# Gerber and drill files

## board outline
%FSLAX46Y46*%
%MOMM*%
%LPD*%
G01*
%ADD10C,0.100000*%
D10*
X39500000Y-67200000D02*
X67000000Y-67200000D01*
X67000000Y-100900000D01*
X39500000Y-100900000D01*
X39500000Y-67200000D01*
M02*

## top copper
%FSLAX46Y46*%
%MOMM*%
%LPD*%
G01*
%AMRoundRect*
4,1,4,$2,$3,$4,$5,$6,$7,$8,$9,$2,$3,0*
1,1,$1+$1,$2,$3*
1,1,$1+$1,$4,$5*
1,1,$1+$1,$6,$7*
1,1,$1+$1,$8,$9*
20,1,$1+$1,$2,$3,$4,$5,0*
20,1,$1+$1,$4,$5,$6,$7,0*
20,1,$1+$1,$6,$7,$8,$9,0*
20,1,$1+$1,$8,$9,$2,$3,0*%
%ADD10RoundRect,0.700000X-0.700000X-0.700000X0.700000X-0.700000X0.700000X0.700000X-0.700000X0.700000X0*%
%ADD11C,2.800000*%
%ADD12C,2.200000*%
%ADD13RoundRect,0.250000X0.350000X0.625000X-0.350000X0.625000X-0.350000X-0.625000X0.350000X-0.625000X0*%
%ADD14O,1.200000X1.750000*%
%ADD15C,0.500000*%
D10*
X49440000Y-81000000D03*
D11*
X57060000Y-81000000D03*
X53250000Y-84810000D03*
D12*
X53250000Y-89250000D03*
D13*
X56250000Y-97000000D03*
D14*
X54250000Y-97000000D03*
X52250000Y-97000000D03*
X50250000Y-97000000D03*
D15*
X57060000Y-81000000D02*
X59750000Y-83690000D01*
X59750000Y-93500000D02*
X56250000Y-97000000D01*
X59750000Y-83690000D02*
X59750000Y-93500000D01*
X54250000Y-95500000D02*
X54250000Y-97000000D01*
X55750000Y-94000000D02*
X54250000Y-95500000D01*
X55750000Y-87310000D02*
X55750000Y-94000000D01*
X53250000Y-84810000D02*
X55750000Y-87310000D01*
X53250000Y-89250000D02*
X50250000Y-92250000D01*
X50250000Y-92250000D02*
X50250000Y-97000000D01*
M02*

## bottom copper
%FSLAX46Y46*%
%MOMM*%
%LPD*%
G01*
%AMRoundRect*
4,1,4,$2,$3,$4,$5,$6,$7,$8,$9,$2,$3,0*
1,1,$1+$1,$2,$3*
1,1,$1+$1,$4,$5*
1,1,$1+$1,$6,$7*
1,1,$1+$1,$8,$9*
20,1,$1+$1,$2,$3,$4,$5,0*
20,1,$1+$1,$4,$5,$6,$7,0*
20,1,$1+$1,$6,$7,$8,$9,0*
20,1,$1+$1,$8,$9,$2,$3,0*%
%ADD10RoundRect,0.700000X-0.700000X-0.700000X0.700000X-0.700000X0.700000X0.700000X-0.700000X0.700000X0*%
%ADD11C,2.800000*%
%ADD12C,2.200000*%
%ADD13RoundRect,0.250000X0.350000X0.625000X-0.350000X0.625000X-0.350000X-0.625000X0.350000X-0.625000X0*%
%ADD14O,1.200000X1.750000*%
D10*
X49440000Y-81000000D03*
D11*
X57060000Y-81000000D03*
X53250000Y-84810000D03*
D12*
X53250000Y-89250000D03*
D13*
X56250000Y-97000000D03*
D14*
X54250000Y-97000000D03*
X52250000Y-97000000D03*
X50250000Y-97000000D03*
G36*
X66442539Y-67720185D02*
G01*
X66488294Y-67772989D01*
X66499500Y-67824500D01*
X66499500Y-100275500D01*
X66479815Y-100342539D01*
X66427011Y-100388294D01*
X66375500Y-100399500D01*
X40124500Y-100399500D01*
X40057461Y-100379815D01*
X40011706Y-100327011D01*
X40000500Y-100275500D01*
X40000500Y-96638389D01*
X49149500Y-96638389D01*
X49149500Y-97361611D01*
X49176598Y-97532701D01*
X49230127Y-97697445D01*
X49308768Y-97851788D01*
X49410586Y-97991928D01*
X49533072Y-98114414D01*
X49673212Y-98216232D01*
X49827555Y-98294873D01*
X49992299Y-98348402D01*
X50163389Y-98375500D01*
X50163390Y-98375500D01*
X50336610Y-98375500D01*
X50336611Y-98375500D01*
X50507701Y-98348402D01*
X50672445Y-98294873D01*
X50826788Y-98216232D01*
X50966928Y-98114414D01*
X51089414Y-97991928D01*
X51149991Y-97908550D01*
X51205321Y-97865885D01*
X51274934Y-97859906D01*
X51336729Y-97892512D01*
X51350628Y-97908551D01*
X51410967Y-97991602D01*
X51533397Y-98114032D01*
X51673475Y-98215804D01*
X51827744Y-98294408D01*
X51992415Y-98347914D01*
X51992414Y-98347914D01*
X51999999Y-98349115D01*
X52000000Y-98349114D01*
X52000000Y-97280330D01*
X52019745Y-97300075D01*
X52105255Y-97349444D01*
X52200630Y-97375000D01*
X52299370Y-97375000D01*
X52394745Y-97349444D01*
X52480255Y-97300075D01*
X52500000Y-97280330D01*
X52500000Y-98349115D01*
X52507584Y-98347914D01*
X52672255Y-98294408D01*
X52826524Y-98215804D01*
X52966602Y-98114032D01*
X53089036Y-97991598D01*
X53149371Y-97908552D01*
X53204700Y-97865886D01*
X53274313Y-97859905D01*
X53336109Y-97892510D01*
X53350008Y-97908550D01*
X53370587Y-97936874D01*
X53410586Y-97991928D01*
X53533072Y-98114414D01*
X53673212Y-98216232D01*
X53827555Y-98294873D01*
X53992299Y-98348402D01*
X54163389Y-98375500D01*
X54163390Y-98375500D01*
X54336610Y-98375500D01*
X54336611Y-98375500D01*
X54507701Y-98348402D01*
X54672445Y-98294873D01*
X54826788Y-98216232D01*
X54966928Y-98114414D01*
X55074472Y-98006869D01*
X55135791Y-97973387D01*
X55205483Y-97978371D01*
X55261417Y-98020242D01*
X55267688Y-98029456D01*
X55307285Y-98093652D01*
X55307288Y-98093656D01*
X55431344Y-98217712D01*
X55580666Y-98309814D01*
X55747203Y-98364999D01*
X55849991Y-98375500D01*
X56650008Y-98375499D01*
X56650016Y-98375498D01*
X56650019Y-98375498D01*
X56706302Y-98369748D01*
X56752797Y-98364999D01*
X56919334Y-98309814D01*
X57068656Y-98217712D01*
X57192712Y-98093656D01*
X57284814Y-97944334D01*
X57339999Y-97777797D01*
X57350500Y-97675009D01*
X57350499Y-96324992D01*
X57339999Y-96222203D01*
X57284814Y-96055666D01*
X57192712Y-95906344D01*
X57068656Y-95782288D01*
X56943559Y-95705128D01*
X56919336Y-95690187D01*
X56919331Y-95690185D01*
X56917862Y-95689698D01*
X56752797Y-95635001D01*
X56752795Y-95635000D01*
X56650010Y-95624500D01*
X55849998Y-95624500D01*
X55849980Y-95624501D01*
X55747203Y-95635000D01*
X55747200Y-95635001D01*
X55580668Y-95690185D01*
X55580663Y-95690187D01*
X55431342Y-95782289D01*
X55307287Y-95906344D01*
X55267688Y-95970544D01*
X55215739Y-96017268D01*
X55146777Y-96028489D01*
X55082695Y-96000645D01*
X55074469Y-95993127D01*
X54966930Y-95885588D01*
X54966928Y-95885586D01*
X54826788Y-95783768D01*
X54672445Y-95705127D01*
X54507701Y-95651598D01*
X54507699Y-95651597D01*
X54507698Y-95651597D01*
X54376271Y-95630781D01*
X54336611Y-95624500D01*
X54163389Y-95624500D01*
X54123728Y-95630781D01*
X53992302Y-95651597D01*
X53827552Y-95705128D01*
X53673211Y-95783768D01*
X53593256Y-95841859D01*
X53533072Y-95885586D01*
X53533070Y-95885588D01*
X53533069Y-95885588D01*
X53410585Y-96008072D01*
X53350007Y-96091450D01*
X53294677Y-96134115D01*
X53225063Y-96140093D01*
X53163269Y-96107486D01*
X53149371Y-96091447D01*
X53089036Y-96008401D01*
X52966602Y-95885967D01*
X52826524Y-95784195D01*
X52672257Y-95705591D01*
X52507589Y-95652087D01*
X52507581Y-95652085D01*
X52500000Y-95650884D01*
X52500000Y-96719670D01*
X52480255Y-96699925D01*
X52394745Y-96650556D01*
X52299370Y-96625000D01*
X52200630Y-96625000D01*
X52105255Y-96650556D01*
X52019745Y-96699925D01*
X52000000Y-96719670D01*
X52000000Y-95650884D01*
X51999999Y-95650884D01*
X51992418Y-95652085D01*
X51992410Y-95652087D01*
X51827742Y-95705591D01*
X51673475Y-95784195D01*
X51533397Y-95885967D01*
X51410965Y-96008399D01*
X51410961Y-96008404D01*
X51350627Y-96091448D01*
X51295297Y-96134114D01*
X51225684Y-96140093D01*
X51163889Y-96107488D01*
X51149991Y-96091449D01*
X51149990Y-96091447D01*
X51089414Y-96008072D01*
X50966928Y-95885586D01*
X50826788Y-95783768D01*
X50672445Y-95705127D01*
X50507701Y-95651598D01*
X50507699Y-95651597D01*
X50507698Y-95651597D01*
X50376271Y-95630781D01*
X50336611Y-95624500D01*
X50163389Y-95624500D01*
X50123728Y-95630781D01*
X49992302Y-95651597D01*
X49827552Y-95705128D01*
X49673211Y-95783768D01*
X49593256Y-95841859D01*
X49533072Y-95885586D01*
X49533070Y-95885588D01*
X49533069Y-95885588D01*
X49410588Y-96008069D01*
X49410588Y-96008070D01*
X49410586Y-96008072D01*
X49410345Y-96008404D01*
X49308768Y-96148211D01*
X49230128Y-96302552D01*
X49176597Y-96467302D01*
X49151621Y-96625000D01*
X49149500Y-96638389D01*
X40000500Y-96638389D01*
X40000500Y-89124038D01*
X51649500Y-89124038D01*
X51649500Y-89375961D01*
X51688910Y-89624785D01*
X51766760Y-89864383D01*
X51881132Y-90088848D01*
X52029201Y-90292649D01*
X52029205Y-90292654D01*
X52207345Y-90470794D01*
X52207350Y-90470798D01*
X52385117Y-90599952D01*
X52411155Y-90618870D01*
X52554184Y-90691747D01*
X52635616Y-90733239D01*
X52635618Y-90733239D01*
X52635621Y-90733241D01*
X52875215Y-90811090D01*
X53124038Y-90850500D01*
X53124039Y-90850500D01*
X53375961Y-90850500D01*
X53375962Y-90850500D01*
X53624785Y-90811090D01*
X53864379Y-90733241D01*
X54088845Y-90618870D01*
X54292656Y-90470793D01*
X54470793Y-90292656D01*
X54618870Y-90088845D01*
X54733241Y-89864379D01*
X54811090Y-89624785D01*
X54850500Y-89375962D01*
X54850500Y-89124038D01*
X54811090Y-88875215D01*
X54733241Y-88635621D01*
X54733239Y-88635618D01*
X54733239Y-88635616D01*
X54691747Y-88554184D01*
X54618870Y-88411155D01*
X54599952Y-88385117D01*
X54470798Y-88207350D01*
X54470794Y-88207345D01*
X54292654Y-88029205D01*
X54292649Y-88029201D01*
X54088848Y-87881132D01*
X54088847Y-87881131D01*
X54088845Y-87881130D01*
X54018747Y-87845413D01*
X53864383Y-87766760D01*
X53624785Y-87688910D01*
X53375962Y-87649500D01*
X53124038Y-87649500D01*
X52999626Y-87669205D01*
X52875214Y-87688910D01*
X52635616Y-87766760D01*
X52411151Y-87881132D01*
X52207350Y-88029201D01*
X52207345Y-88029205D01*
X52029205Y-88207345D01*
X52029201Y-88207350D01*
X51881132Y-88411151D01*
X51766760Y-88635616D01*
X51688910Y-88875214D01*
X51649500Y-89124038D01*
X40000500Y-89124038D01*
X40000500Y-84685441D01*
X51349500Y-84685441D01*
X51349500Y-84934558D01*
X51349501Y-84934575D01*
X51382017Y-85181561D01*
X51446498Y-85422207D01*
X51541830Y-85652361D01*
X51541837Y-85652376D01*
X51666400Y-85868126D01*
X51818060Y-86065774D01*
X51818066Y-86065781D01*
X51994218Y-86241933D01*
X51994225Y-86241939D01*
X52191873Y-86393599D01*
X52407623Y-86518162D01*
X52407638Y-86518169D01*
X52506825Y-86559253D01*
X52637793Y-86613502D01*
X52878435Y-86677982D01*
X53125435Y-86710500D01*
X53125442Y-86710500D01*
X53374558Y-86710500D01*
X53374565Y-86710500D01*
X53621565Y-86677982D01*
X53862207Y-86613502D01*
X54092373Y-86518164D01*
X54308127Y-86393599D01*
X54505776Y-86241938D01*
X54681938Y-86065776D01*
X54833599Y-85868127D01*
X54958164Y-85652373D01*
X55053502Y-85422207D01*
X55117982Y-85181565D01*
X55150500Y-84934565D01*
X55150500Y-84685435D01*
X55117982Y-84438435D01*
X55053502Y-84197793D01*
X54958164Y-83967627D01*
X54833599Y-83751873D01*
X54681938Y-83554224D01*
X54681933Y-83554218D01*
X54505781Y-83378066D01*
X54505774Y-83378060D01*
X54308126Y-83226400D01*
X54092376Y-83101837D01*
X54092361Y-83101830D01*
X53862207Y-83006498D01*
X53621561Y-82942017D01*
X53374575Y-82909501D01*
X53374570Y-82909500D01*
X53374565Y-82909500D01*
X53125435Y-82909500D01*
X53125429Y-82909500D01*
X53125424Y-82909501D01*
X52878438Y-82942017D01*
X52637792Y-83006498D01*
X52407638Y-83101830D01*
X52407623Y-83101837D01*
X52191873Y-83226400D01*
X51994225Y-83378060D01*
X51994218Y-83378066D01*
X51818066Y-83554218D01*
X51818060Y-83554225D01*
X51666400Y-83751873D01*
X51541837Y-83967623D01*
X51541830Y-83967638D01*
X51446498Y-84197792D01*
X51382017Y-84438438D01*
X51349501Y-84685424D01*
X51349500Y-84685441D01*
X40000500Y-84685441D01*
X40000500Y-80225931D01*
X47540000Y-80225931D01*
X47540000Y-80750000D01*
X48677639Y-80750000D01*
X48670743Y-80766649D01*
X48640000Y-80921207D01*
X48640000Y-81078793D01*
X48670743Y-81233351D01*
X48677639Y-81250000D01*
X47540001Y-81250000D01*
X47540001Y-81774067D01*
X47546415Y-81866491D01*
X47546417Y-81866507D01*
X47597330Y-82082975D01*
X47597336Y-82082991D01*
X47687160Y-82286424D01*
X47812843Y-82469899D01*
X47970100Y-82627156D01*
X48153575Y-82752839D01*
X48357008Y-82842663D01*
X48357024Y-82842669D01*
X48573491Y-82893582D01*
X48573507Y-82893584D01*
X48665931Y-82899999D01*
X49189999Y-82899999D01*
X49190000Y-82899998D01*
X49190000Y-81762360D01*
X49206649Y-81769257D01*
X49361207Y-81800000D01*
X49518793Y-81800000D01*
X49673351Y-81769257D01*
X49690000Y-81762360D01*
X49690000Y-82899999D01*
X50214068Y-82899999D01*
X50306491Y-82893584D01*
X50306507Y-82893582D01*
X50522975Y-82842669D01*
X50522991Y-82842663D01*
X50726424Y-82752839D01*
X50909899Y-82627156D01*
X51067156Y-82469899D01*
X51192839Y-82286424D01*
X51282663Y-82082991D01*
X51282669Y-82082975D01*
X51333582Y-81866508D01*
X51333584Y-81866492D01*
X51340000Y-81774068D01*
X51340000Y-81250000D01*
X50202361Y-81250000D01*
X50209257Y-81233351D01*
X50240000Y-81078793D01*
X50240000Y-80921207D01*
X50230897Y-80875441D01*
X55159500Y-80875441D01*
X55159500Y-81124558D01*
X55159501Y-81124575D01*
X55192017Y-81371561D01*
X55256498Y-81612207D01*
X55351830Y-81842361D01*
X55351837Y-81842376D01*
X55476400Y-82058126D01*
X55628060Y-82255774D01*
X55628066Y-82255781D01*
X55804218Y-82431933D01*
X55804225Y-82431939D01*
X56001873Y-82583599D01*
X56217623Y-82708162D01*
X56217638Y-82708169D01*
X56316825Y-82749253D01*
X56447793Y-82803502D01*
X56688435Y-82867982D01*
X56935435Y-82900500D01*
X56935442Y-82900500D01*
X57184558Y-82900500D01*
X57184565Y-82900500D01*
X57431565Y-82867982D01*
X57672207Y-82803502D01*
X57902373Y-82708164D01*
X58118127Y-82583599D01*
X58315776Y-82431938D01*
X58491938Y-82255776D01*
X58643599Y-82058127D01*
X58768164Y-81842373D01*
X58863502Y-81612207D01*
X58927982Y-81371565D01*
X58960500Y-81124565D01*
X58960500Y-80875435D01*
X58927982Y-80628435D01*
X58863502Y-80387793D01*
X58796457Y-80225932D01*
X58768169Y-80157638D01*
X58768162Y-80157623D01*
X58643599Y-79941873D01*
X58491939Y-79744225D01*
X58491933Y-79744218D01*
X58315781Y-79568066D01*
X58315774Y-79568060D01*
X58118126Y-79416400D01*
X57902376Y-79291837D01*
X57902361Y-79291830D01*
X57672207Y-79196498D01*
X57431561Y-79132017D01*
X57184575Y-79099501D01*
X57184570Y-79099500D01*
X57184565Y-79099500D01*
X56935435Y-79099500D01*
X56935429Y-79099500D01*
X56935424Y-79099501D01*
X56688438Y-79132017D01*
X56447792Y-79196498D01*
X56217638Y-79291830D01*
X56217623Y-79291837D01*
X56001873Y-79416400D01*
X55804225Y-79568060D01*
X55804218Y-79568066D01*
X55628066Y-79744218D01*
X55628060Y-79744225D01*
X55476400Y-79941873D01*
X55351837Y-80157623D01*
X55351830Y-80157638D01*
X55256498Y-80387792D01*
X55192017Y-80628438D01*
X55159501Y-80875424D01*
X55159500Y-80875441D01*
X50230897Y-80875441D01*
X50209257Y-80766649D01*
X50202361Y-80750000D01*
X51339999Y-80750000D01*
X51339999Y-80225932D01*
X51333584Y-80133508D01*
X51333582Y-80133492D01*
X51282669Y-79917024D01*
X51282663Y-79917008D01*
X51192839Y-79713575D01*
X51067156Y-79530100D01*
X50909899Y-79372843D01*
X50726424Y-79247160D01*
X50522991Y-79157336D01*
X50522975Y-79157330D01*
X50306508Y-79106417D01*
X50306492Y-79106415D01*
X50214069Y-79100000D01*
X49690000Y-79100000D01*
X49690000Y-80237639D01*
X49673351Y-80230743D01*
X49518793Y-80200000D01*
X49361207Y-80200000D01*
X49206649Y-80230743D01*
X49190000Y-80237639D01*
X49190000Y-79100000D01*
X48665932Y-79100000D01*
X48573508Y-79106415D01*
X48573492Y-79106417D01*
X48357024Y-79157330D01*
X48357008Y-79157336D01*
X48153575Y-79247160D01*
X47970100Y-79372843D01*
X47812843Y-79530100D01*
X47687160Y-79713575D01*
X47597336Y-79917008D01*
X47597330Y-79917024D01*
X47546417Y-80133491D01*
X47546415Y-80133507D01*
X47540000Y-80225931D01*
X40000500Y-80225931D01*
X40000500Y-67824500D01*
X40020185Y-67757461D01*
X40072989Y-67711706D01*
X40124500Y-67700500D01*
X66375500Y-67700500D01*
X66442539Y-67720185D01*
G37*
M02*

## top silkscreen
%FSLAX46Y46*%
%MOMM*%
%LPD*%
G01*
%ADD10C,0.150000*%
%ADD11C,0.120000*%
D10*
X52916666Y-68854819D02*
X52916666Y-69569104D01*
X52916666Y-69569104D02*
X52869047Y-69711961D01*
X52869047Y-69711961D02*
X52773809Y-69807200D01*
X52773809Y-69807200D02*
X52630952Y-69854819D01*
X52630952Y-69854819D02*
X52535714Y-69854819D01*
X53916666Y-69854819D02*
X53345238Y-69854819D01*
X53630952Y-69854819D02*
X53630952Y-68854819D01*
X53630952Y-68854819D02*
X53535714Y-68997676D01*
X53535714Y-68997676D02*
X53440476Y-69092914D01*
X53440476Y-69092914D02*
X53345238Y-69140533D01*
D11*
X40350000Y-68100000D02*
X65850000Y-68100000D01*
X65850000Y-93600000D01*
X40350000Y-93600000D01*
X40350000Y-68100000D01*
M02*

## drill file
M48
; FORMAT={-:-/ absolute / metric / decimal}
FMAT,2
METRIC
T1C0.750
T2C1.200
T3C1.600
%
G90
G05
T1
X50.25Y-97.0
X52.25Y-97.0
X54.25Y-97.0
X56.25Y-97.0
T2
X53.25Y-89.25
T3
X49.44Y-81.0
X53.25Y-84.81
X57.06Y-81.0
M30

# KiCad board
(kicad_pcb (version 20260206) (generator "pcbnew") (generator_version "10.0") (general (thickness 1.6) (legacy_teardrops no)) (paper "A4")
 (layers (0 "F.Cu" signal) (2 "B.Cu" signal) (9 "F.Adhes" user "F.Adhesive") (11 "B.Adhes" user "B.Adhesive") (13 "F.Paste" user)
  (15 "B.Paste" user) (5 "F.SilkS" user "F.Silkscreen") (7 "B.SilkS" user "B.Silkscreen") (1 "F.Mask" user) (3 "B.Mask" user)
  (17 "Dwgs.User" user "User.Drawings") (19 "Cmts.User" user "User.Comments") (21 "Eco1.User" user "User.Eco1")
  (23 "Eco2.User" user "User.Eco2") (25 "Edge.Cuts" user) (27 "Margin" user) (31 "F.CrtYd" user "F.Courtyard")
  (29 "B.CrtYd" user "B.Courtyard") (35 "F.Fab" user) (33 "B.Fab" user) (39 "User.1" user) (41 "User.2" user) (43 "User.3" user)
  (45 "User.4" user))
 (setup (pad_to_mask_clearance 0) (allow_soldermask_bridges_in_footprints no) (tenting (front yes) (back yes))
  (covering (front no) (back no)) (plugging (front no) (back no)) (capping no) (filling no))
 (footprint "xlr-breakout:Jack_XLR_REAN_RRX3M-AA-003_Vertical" (layer "F.Cu") (at 53.25 81)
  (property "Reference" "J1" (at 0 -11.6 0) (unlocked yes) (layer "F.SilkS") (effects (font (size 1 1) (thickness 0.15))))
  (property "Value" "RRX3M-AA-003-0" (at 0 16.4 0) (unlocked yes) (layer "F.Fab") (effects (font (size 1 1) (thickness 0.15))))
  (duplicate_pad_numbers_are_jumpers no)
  (fp_rect (start -12.9 -12.9) (end 12.6 12.6) (stroke (width 0.12) (type solid)) (fill no) (layer "F.SilkS"))
  (pad "1" thru_hole roundrect (at -3.81 0) (size 2.8 2.8) (drill 1.6) (layers "*.Cu" "*.Mask") (remove_unused_layers no)
   (roundrect_rratio 0.25) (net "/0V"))
  (pad "2" thru_hole circle (at 3.81 0) (size 2.8 2.8) (drill 1.6) (layers "*.Cu" "*.Mask") (remove_unused_layers no) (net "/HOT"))
  (pad "3" thru_hole circle (at 0 3.81) (size 2.8 2.8) (drill 1.6) (layers "*.Cu" "*.Mask") (remove_unused_layers no) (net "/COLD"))
  (pad "G" thru_hole circle (at 0 8.25) (size 2.2 2.2) (drill 1.2) (layers "*.Cu" "*.Mask") (remove_unused_layers no) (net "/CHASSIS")))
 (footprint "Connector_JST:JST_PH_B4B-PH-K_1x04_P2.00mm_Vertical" (layer "B.Cu") (at 56.25 97 180)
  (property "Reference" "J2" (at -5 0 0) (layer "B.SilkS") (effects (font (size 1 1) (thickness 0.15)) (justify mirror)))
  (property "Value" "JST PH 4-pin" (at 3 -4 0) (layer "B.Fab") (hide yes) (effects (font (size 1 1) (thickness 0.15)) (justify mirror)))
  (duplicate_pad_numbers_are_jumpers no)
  (pad "1" thru_hole roundrect (at 0 0 180) (size 1.2 1.75) (drill 0.75) (layers "*.Cu" "*.Mask") (remove_unused_layers no)
   (roundrect_rratio 0.208333) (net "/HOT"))
  (pad "2" thru_hole oval (at 2 0 180) (size 1.2 1.75) (drill 0.75) (layers "*.Cu" "*.Mask") (remove_unused_layers no) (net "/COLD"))
  (pad "3" thru_hole oval (at 4 0 180) (size 1.2 1.75) (drill 0.75) (layers "*.Cu" "*.Mask") (remove_unused_layers no) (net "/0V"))
  (pad "4" thru_hole oval (at 6 0 180) (size 1.2 1.75) (drill 0.75) (layers "*.Cu" "*.Mask") (remove_unused_layers no) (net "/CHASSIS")))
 (gr_rect (start 39.5 67.2) (end 67 100.9) (stroke (width 0.1) (type default)) (fill no) (layer "Edge.Cuts"))
 (segment (start 57.06 81) (end 59.75 83.69) (width 0.5) (layer "F.Cu") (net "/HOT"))
 (segment (start 59.75 93.5) (end 56.25 97) (width 0.5) (layer "F.Cu") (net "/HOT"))
 (segment (start 59.75 83.69) (end 59.75 93.5) (width 0.5) (layer "F.Cu") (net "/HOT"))
 (segment (start 54.25 95.5) (end 54.25 97) (width 0.5) (layer "F.Cu") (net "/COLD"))
 (segment (start 55.75 94) (end 54.25 95.5) (width 0.5) (layer "F.Cu") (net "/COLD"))
 (segment (start 55.75 87.31) (end 55.75 94) (width 0.5) (layer "F.Cu") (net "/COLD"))
 (segment (start 53.25 84.81) (end 55.75 87.31) (width 0.5) (layer "F.Cu") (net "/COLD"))
 (segment (start 53.25 89.25) (end 50.25 92.25) (width 0.5) (layer "F.Cu") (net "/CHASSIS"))
 (segment (start 50.25 92.25) (end 50.25 97) (width 0.5) (layer "F.Cu") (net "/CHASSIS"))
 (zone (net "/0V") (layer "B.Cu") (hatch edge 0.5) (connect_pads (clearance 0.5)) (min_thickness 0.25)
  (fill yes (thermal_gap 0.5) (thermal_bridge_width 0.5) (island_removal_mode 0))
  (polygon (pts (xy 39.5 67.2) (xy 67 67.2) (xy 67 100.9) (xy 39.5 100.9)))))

